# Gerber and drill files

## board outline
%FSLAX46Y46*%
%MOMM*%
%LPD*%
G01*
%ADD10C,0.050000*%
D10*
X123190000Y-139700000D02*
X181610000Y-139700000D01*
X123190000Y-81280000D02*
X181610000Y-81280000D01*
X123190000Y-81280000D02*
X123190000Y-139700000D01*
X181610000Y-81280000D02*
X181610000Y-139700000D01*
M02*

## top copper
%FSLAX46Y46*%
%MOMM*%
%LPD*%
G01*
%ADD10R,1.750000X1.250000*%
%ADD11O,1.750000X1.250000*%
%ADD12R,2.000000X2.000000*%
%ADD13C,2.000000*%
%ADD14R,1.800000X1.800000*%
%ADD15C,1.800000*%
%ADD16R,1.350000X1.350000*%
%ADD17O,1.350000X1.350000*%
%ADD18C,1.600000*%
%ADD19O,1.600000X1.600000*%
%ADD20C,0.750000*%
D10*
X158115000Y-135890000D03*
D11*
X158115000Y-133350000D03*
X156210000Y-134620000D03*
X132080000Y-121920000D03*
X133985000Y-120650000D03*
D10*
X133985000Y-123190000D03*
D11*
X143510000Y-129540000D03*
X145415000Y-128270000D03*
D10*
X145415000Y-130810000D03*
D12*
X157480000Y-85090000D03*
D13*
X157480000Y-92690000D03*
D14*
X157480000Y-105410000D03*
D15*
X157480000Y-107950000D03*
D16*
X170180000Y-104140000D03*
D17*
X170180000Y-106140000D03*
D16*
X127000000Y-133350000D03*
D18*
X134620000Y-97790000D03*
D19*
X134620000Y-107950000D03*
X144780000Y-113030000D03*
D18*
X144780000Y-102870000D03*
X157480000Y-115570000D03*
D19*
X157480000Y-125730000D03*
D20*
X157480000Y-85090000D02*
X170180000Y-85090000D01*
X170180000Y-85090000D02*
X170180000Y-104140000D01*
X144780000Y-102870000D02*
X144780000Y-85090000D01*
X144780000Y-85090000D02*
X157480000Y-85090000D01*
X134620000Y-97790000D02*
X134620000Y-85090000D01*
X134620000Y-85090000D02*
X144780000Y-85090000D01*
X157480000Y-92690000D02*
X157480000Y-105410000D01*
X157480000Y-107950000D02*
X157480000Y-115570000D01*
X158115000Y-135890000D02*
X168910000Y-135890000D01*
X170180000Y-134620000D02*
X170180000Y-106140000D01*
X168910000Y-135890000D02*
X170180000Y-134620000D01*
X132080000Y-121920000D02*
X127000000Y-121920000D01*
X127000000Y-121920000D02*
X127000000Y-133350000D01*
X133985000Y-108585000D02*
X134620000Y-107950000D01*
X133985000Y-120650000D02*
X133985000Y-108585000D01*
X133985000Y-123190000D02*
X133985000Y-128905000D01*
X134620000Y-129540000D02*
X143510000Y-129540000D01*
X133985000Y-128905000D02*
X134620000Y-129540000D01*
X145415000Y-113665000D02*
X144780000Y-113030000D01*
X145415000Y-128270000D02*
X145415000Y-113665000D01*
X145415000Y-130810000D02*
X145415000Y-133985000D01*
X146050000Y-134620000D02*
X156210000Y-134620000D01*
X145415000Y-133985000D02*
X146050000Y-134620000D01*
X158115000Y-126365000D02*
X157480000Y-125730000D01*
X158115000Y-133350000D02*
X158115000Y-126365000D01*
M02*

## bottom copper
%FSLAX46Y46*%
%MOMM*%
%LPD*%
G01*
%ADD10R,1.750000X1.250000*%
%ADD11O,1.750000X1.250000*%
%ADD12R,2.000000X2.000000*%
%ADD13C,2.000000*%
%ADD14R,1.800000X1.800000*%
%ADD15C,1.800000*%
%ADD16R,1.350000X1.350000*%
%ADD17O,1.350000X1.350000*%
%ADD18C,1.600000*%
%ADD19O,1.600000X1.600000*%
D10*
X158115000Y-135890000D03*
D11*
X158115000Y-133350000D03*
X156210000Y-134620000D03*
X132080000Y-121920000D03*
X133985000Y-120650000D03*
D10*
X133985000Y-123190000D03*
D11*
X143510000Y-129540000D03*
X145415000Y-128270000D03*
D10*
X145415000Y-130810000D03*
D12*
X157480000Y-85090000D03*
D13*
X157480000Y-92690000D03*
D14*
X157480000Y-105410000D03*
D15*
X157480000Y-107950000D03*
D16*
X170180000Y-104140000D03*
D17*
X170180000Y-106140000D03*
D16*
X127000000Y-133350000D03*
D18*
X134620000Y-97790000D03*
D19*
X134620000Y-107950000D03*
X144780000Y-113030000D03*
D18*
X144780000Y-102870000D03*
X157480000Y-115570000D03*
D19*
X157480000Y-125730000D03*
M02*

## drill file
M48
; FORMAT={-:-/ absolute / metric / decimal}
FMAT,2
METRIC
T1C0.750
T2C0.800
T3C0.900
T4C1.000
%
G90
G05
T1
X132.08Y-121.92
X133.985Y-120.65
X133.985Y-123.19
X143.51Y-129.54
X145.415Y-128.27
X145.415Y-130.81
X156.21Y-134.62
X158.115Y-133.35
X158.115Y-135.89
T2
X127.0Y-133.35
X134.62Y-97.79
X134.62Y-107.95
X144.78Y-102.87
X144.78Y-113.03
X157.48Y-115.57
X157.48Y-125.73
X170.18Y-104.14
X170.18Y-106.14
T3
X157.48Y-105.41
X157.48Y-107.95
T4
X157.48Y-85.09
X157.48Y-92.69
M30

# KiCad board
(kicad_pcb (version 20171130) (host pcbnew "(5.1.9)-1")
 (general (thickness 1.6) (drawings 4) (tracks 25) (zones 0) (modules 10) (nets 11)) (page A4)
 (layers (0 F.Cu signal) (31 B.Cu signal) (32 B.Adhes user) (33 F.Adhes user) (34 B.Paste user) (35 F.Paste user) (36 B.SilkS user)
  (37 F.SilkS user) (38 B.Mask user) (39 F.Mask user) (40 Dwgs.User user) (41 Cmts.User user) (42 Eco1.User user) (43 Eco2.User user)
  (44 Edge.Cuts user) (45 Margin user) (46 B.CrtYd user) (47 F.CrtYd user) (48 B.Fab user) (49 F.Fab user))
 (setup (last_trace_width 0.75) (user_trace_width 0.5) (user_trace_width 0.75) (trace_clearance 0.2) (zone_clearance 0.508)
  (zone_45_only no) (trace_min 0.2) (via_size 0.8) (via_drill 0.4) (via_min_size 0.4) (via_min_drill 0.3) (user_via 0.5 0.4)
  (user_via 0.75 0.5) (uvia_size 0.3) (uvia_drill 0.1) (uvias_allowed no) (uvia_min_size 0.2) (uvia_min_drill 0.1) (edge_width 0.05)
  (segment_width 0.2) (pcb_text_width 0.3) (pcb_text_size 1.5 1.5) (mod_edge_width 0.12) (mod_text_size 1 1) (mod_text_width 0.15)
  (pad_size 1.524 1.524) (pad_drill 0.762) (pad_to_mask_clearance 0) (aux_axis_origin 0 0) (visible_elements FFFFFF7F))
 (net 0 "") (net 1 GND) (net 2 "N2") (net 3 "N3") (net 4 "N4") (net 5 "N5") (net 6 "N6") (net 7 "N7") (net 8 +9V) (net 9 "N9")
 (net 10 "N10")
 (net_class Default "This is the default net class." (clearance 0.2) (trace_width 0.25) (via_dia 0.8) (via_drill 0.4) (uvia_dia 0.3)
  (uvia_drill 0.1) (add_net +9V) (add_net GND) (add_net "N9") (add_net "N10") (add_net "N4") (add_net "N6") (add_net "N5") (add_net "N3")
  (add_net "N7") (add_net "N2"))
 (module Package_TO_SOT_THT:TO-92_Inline (layer F.Cu) (at 157.48 135.89 90)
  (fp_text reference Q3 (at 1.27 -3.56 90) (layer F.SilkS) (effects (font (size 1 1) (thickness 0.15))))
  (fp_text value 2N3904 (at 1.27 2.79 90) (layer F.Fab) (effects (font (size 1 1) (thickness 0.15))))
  (pad 1 thru_hole rect (at 0 0.635 90) (size 1.25 1.75) (drill 0.75) (layers *.Cu *.Mask) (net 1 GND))
  (pad 3 thru_hole oval (at 2.54 0.635 90) (size 1.25 1.75) (drill 0.75) (layers *.Cu *.Mask) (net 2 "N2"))
  (pad 2 thru_hole oval (at 1.27 -1.27 90) (size 1.25 1.75) (drill 0.75) (layers *.Cu *.Mask) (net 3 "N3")))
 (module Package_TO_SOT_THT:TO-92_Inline (layer F.Cu) (at 133.35 123.19 90)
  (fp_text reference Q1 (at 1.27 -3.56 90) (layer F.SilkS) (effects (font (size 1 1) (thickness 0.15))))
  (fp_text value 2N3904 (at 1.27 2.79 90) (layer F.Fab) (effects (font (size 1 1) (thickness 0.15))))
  (pad 2 thru_hole oval (at 1.27 -1.27 90) (size 1.25 1.75) (drill 0.75) (layers *.Cu *.Mask) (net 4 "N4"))
  (pad 3 thru_hole oval (at 2.54 0.635 90) (size 1.25 1.75) (drill 0.75) (layers *.Cu *.Mask) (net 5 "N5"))
  (pad 1 thru_hole rect (at 0 0.635 90) (size 1.25 1.75) (drill 0.75) (layers *.Cu *.Mask) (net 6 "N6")))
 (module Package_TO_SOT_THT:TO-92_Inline (layer F.Cu) (at 144.78 130.81 90)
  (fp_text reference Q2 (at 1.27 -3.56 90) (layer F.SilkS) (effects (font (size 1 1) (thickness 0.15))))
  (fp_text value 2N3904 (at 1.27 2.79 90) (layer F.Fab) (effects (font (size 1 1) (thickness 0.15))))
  (pad 2 thru_hole oval (at 1.27 -1.27 90) (size 1.25 1.75) (drill 0.75) (layers *.Cu *.Mask) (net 6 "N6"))
  (pad 3 thru_hole oval (at 2.54 0.635 90) (size 1.25 1.75) (drill 0.75) (layers *.Cu *.Mask) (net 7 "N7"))
  (pad 1 thru_hole rect (at 0 0.635 90) (size 1.25 1.75) (drill 0.75) (layers *.Cu *.Mask) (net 3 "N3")))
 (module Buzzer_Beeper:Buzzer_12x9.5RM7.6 (layer F.Cu) (at 157.48 85.09 270)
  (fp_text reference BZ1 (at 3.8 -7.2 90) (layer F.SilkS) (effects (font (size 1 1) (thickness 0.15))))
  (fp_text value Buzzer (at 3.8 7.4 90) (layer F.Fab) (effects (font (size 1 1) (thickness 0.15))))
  (pad 1 thru_hole rect (at 0 0 270) (size 2 2) (drill 1) (layers *.Cu *.Mask) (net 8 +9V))
  (pad 2 thru_hole circle (at 7.6 0 270) (size 2 2) (drill 1) (layers *.Cu *.Mask) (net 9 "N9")))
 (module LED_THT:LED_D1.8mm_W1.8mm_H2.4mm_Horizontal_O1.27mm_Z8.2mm (layer F.Cu) (at 157.48 105.41 270)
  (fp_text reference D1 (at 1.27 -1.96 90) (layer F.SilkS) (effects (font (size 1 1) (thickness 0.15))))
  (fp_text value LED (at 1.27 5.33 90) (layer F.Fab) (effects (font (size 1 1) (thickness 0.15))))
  (pad 1 thru_hole rect (at 0 0 270) (size 1.8 1.8) (drill 0.9) (layers *.Cu *.Mask) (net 9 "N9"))
  (pad 2 thru_hole circle (at 2.54 0 270) (size 1.8 1.8) (drill 0.9) (layers *.Cu *.Mask) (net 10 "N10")))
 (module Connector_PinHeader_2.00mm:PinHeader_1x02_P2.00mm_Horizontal (layer F.Cu) (at 170.18 104.14)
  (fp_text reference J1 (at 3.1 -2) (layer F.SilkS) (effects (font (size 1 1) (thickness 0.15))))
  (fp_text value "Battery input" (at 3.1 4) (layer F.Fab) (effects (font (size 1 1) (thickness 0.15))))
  (pad 1 thru_hole rect (at 0 0) (size 1.35 1.35) (drill 0.8) (layers *.Cu *.Mask) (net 8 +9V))
  (pad 2 thru_hole oval (at 0 2) (size 1.35 1.35) (drill 0.8) (layers *.Cu *.Mask) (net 1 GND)))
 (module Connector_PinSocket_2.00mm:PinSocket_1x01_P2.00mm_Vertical (layer F.Cu) (at 127 133.35)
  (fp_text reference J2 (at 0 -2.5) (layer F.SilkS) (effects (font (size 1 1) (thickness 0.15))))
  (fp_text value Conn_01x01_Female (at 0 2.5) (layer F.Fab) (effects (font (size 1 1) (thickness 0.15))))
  (pad 1 thru_hole rect (at 0 0) (size 1.35 1.35) (drill 0.8) (layers *.Cu *.Mask) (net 4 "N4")))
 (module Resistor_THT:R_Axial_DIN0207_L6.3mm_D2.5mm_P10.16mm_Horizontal (layer F.Cu) (at 134.62 97.79 270)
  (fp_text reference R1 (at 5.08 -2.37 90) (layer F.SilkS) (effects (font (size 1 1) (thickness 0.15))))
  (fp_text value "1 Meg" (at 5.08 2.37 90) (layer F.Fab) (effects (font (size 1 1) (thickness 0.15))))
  (pad 1 thru_hole circle (at 0 0 270) (size 1.6 1.6) (drill 0.8) (layers *.Cu *.Mask) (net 8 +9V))
  (pad 2 thru_hole oval (at 10.16 0 270) (size 1.6 1.6) (drill 0.8) (layers *.Cu *.Mask) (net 5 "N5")))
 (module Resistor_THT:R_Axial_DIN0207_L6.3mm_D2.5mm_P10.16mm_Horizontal (layer F.Cu) (at 144.78 102.87 270)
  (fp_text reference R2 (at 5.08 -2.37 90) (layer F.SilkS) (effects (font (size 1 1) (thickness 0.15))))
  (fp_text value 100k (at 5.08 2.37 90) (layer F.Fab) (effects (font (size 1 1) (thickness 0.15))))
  (pad 2 thru_hole oval (at 10.16 0 270) (size 1.6 1.6) (drill 0.8) (layers *.Cu *.Mask) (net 7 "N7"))
  (pad 1 thru_hole circle (at 0 0 270) (size 1.6 1.6) (drill 0.8) (layers *.Cu *.Mask) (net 8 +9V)))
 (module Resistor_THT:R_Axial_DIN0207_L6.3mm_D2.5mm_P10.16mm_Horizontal (layer F.Cu) (at 157.48 115.57 270)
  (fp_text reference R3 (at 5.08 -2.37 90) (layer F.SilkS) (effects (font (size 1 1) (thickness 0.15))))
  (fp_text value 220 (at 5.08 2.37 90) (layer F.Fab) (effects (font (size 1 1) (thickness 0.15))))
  (pad 1 thru_hole circle (at 0 0 270) (size 1.6 1.6) (drill 0.8) (layers *.Cu *.Mask) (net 10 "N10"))
  (pad 2 thru_hole oval (at 10.16 0 270) (size 1.6 1.6) (drill 0.8) (layers *.Cu *.Mask) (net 2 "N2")))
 (gr_line (start 123.19 139.7) (end 181.61 139.7) (layer Edge.Cuts) (width 0.05))
 (gr_line (start 123.19 81.28) (end 181.61 81.28) (layer Edge.Cuts) (width 0.05))
 (gr_line (start 123.19 81.28) (end 123.19 139.7) (layer Edge.Cuts) (width 0.05))
 (gr_line (start 181.61 81.28) (end 181.61 139.7) (layer Edge.Cuts) (width 0.05))
 (segment (start 157.48 85.09) (end 170.18 85.09) (width 0.75) (layer F.Cu) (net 8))
 (segment (start 170.18 85.09) (end 170.18 104.14) (width 0.75) (layer F.Cu) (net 8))
 (segment (start 144.78 102.87) (end 144.78 85.09) (width 0.75) (layer F.Cu) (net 8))
 (segment (start 144.78 85.09) (end 157.48 85.09) (width 0.75) (layer F.Cu) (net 8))
 (segment (start 134.62 97.79) (end 134.62 85.09) (width 0.75) (layer F.Cu) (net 8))
 (segment (start 134.62 85.09) (end 144.78 85.09) (width 0.75) (layer F.Cu) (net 8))
 (segment (start 157.48 92.69) (end 157.48 105.41) (width 0.75) (layer F.Cu) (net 9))
 (segment (start 157.48 107.95) (end 157.48 115.57) (width 0.75) (layer F.Cu) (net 10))
 (segment (start 158.115 135.89) (end 168.91 135.89) (width 0.75) (layer F.Cu) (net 1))
 (segment (start 170.18 134.62) (end 170.18 106.14) (width 0.75) (layer F.Cu) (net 1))
 (segment (start 168.91 135.89) (end 170.18 134.62) (width 0.75) (layer F.Cu) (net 1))
 (segment (start 132.08 121.92) (end 127 121.92) (width 0.75) (layer F.Cu) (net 4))
 (segment (start 127 121.92) (end 127 133.35) (width 0.75) (layer F.Cu) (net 4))
 (segment (start 133.985 108.585) (end 134.62 107.95) (width 0.75) (layer F.Cu) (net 5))
 (segment (start 133.985 120.65) (end 133.985 108.585) (width 0.75) (layer F.Cu) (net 5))
 (segment (start 133.985 123.19) (end 133.985 128.905) (width 0.75) (layer F.Cu) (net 6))
 (segment (start 134.62 129.54) (end 143.51 129.54) (width 0.75) (layer F.Cu) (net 6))
 (segment (start 133.985 128.905) (end 134.62 129.54) (width 0.75) (layer F.Cu) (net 6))
 (segment (start 145.415 113.665) (end 144.78 113.03) (width 0.75) (layer F.Cu) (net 7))
 (segment (start 145.415 128.27) (end 145.415 113.665) (width 0.75) (layer F.Cu) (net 7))
 (segment (start 145.415 130.81) (end 145.415 133.985) (width 0.75) (layer F.Cu) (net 3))
 (segment (start 146.05 134.62) (end 156.21 134.62) (width 0.75) (layer F.Cu) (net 3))
 (segment (start 145.415 133.985) (end 146.05 134.62) (width 0.75) (layer F.Cu) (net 3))
 (segment (start 158.115 126.365) (end 157.48 125.73) (width 0.75) (layer F.Cu) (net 2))
 (segment (start 158.115 133.35) (end 158.115 126.365) (width 0.75) (layer F.Cu) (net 2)))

